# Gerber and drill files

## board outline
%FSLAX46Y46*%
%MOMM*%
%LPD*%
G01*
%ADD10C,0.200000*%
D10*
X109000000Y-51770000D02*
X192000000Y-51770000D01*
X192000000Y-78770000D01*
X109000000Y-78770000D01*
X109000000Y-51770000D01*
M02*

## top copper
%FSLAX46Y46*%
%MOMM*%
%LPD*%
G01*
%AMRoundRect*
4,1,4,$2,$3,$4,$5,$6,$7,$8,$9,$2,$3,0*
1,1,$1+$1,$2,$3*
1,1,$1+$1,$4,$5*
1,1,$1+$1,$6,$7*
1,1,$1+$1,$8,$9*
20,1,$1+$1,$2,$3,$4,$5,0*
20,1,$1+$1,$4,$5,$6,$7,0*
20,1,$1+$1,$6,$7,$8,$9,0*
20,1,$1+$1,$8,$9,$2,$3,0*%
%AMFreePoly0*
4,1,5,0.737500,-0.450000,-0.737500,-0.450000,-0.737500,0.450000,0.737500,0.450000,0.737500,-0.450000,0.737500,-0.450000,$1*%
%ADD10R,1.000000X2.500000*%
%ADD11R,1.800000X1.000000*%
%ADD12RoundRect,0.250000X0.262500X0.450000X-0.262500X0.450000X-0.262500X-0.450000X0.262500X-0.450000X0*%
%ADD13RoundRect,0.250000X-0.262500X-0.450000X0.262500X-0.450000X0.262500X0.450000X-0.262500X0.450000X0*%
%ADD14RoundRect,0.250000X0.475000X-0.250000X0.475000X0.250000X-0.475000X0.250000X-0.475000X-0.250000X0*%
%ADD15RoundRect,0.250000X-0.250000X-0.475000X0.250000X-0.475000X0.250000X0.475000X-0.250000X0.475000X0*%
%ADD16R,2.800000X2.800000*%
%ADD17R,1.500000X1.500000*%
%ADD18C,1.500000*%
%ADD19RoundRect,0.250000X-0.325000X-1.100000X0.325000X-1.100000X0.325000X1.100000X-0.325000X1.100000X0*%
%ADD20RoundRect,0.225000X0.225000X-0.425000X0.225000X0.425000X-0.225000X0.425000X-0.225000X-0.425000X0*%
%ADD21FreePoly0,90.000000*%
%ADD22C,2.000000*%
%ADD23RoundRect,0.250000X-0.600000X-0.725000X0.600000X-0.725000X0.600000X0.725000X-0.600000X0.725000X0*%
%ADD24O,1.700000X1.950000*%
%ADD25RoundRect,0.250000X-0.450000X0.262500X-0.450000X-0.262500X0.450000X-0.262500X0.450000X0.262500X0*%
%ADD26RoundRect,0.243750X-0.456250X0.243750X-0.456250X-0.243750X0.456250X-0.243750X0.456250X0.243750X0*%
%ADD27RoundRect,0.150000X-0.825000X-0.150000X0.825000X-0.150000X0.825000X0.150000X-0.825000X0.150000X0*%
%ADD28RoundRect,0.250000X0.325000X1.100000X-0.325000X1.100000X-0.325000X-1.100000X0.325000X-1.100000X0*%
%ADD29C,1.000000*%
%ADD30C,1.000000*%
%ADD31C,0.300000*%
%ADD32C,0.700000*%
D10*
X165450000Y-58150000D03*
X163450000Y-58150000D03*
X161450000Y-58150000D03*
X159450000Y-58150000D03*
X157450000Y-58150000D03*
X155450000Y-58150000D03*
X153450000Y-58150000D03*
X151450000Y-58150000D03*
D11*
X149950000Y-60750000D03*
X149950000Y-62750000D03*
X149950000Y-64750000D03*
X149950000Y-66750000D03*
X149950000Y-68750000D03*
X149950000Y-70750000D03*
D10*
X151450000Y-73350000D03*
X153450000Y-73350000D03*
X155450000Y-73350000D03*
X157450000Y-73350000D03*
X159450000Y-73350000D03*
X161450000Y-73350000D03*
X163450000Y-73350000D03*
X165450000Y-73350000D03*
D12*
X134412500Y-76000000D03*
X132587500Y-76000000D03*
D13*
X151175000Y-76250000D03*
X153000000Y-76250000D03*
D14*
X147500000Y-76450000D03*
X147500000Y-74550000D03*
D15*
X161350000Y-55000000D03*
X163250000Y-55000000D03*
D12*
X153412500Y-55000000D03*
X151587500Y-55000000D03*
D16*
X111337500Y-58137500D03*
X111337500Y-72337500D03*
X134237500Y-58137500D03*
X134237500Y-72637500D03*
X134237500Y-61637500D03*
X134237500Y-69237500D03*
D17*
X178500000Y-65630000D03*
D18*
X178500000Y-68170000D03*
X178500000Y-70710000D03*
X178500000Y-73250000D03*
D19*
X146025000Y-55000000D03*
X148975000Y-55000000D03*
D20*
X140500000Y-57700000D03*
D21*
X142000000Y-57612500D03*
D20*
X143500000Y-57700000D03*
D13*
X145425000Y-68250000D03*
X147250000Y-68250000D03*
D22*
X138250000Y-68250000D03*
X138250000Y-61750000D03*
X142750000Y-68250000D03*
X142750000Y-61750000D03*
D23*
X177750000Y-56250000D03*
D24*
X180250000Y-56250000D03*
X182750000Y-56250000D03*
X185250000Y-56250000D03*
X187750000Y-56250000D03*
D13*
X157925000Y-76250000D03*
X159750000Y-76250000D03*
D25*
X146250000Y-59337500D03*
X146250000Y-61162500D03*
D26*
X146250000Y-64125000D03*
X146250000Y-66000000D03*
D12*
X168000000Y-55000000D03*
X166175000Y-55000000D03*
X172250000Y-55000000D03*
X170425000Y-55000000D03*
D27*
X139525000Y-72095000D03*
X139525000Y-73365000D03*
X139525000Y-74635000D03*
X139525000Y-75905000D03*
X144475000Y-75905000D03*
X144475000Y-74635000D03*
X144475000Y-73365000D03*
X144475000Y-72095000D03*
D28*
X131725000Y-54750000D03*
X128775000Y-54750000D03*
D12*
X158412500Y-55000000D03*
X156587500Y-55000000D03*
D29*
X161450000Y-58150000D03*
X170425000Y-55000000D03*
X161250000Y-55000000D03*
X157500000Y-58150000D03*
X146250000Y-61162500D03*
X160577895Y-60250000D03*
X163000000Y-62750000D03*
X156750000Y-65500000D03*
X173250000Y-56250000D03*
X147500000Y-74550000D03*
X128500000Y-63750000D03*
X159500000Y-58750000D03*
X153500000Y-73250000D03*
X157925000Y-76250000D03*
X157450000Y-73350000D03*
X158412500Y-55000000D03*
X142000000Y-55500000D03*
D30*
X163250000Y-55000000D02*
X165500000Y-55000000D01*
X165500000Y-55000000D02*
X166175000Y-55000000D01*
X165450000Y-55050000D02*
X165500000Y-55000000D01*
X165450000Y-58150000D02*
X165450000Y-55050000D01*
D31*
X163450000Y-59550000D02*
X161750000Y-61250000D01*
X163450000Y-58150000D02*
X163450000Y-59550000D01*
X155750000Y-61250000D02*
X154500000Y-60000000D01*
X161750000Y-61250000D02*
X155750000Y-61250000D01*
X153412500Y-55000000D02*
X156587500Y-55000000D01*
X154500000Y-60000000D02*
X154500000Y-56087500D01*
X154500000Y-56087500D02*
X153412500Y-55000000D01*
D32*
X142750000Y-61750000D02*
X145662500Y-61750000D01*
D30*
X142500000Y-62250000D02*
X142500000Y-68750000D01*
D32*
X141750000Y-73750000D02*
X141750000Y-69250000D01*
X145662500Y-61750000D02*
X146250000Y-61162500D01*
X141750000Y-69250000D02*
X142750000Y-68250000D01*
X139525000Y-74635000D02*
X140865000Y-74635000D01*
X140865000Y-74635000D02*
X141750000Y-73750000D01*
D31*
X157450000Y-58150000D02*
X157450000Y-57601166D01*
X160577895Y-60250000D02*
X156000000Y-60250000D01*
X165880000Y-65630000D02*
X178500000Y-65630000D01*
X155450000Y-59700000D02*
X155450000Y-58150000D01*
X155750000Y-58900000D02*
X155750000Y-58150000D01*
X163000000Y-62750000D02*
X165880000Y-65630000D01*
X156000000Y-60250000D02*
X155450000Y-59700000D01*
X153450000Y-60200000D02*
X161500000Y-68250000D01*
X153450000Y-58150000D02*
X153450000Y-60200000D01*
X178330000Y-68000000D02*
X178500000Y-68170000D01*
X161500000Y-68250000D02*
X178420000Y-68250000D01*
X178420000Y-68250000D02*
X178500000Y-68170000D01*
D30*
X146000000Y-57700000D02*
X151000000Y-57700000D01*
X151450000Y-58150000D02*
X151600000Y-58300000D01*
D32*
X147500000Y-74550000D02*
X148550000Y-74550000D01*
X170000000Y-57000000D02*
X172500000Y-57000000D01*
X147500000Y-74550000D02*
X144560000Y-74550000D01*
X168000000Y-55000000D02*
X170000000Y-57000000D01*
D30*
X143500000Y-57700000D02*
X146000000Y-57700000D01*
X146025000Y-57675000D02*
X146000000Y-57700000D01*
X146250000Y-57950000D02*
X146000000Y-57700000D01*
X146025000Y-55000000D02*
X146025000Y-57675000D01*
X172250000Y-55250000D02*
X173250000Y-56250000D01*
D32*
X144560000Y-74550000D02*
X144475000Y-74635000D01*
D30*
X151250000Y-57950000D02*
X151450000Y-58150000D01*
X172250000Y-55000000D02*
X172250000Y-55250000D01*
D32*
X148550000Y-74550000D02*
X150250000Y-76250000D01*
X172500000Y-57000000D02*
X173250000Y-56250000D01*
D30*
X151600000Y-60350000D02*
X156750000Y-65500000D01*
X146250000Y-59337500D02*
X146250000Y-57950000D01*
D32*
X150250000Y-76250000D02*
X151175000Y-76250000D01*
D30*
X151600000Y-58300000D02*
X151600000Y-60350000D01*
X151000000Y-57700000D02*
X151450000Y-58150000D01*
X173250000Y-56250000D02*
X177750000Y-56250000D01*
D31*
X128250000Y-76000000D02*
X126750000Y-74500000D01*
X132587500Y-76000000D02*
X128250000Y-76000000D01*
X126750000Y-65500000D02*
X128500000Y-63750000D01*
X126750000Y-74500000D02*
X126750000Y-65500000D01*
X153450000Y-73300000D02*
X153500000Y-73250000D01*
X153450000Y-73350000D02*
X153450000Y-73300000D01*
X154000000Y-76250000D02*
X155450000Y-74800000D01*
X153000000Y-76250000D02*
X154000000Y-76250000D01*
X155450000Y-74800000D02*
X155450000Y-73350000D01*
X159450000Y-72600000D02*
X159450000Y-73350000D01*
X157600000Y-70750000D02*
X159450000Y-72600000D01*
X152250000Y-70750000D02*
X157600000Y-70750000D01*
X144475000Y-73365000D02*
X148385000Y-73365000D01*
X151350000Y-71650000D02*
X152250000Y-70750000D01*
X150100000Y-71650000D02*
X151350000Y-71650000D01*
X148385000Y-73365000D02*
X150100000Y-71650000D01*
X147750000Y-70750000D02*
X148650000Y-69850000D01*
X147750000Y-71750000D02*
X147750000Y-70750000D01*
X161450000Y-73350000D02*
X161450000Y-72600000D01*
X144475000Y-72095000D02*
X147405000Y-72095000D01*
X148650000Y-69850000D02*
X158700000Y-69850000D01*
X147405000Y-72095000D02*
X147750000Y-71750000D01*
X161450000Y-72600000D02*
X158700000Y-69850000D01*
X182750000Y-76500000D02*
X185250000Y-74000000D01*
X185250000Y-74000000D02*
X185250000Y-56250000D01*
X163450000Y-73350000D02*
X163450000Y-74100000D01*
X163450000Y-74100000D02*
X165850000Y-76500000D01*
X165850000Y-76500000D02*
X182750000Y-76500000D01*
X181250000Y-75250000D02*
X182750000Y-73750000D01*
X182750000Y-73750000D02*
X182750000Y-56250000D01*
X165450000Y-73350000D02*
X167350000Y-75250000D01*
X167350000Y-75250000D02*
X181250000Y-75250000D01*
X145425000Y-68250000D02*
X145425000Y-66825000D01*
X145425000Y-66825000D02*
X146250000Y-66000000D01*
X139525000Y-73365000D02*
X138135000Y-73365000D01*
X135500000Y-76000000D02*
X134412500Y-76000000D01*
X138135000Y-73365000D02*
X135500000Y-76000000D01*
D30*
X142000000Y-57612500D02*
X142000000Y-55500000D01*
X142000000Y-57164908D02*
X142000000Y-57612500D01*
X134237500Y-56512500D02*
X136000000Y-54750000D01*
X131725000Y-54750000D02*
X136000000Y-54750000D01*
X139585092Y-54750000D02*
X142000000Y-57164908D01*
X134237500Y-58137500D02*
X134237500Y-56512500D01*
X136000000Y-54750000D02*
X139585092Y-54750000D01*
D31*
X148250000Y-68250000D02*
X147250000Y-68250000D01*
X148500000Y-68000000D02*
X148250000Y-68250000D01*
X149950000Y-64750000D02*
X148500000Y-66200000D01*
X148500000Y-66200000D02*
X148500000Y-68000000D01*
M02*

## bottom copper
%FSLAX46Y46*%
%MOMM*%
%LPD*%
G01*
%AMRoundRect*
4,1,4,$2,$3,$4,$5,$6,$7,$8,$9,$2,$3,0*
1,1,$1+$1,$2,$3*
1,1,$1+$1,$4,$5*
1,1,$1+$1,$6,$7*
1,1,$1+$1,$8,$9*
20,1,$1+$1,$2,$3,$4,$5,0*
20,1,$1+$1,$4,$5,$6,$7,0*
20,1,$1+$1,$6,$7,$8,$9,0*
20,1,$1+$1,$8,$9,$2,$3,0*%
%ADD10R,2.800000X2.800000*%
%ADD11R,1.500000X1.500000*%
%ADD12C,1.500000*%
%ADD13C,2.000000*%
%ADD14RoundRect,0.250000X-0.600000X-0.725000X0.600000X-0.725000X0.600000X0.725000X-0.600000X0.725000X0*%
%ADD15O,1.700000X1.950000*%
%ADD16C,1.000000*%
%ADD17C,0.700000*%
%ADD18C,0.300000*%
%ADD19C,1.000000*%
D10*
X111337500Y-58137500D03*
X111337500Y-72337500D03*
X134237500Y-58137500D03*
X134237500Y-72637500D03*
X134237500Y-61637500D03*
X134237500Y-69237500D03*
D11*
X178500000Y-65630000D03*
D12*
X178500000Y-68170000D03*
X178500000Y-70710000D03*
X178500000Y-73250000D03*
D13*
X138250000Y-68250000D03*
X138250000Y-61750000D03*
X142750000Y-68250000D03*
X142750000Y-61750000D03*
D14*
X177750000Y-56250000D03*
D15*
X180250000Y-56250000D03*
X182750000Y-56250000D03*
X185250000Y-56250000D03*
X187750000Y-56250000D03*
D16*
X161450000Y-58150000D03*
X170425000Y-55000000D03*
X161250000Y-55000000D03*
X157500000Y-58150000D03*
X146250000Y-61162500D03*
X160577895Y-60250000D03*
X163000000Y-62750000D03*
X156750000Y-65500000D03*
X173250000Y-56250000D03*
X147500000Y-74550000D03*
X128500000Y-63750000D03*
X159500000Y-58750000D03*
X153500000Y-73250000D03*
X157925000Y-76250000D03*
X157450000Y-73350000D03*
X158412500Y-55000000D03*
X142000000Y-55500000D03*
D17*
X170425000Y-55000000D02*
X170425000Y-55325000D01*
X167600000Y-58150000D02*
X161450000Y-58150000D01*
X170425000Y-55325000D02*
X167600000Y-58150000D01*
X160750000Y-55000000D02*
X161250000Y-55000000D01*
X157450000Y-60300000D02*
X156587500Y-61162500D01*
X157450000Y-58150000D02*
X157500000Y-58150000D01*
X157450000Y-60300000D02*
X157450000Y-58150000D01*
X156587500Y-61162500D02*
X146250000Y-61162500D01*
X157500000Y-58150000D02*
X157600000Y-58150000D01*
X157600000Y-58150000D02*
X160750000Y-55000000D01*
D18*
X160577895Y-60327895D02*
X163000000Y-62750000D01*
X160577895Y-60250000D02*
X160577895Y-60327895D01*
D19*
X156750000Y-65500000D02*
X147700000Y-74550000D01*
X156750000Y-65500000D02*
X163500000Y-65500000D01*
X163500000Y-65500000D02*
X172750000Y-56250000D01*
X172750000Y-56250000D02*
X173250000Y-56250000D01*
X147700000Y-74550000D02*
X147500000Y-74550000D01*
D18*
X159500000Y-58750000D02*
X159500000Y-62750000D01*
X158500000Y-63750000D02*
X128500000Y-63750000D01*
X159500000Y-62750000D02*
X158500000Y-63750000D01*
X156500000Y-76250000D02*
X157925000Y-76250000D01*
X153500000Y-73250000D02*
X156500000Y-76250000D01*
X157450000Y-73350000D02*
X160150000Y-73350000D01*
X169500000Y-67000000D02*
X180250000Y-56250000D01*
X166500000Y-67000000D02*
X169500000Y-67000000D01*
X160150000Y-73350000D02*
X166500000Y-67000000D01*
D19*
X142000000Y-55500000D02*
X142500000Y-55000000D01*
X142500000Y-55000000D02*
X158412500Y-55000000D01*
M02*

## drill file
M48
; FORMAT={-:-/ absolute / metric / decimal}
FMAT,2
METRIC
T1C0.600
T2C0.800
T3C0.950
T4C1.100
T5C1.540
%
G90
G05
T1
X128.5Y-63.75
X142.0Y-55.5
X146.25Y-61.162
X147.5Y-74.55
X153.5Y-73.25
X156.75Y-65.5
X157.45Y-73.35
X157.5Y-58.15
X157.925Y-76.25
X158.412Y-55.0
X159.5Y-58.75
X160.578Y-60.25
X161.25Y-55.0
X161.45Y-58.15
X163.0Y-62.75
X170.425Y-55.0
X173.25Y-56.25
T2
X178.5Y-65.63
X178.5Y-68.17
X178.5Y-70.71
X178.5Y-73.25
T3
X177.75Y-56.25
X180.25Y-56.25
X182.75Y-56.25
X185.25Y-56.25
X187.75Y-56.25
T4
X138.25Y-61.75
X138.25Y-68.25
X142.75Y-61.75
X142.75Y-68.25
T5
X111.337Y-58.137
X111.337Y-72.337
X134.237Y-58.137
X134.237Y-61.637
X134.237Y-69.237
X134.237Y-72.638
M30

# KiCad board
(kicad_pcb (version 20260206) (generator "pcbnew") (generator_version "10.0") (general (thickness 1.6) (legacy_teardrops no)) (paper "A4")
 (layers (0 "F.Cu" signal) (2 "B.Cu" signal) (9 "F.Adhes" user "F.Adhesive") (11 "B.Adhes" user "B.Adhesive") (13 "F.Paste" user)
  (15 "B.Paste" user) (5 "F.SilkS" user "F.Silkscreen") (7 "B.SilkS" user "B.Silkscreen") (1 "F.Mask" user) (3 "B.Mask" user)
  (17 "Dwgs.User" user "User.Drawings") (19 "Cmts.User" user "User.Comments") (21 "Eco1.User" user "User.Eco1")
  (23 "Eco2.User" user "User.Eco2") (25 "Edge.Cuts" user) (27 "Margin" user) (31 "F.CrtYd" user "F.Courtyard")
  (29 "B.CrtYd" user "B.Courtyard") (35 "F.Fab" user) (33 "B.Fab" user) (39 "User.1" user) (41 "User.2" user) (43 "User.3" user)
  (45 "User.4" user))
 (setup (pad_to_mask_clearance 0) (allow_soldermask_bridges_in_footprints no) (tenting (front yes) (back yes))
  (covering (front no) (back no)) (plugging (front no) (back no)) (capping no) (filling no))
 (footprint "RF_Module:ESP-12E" (layer "F.Cu") (at 161.95 65.75 -90)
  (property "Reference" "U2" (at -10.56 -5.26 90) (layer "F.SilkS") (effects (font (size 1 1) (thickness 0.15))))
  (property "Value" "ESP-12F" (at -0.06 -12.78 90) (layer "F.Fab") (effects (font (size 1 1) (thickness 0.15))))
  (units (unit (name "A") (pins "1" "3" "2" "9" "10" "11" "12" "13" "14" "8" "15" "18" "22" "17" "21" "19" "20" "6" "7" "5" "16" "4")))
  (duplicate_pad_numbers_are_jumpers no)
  (pad "1" smd rect (at -7.6 -3.5 270) (size 2.5 1) (layers "F.Cu" "F.Mask" "F.Paste") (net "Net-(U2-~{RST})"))
  (pad "2" smd rect (at -7.6 -1.5 270) (size 2.5 1) (layers "F.Cu" "F.Mask" "F.Paste") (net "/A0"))
  (pad "3" smd rect (at -7.6 0.5 270) (size 2.5 1) (layers "F.Cu" "F.Mask" "F.Paste") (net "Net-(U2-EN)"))
  (pad "4" smd rect (at -7.6 2.5 270) (size 2.5 1) (layers "F.Cu" "F.Mask" "F.Paste") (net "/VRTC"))
  (pad "5" smd rect (at -7.6 4.5 270) (size 2.5 1) (layers "F.Cu" "F.Mask" "F.Paste") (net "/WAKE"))
  (pad "6" smd rect (at -7.6 6.5 270) (size 2.5 1) (layers "F.Cu" "F.Mask" "F.Paste") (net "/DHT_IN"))
  (pad "7" smd rect (at -7.6 8.5 270) (size 2.5 1) (layers "F.Cu" "F.Mask" "F.Paste") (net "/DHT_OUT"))
  (pad "8" smd rect (at -7.6 10.5 270) (size 2.5 1) (layers "F.Cu" "F.Mask" "F.Paste") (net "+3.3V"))
  (pad "9" smd rect (at -5 12 270) (size 1 1.8) (layers "F.Cu" "F.Mask" "F.Paste") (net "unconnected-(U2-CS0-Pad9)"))
  (pad "10" smd rect (at -3 12 270) (size 1 1.8) (layers "F.Cu" "F.Mask" "F.Paste") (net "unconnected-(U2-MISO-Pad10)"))
  (pad "11" smd rect (at -1 12 270) (size 1 1.8) (layers "F.Cu" "F.Mask" "F.Paste") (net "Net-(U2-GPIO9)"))
  (pad "12" smd rect (at 1 12 270) (size 1 1.8) (layers "F.Cu" "F.Mask" "F.Paste") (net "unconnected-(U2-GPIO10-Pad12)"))
  (pad "13" smd rect (at 3 12 270) (size 1 1.8) (layers "F.Cu" "F.Mask" "F.Paste") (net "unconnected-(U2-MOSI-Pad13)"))
  (pad "14" smd rect (at 5 12 270) (size 1 1.8) (layers "F.Cu" "F.Mask" "F.Paste") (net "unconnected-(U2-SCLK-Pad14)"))
  (pad "15" smd rect (at 7.6 10.5 270) (size 2.5 1) (layers "F.Cu" "F.Mask" "F.Paste") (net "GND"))
  (pad "16" smd rect (at 7.6 8.5 270) (size 2.5 1) (layers "F.Cu" "F.Mask" "F.Paste") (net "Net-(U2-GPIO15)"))
  (pad "17" smd rect (at 7.6 6.5 270) (size 2.5 1) (layers "F.Cu" "F.Mask" "F.Paste") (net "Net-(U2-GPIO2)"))
  (pad "18" smd rect (at 7.6 4.5 270) (size 2.5 1) (layers "F.Cu" "F.Mask" "F.Paste") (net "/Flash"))
  (pad "19" smd rect (at 7.6 2.5 270) (size 2.5 1) (layers "F.Cu" "F.Mask" "F.Paste") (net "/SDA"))
  (pad "20" smd rect (at 7.6 0.5 270) (size 2.5 1) (layers "F.Cu" "F.Mask" "F.Paste") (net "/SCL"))
  (pad "21" smd rect (at 7.6 -1.5 270) (size 2.5 1) (layers "F.Cu" "F.Mask" "F.Paste") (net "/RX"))
  (pad "22" smd rect (at 7.6 -3.5 270) (size 2.5 1) (layers "F.Cu" "F.Mask" "F.Paste") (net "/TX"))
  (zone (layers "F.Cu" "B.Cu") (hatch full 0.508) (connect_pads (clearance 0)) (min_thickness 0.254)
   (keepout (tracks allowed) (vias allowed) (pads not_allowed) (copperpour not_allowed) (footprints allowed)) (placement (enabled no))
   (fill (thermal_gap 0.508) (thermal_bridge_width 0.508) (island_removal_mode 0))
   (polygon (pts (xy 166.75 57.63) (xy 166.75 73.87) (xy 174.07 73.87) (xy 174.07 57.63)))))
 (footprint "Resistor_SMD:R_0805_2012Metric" (layer "F.Cu") (at 133.5 76 180)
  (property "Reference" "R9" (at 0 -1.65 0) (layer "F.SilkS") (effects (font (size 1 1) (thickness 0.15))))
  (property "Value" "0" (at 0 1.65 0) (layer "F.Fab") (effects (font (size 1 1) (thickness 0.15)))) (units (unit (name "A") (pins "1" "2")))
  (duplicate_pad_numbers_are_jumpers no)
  (pad "1" smd roundrect (at -0.9125 0 180) (size 1.025 1.4) (layers "F.Cu" "F.Mask" "F.Paste") (roundrect_rratio 0.243902)
   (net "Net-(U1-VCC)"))
  (pad "2" smd roundrect (at 0.9125 0 180) (size 1.025 1.4) (layers "F.Cu" "F.Mask" "F.Paste") (roundrect_rratio 0.243902) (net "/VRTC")))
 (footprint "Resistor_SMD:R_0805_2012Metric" (layer "F.Cu") (at 152.0875 76.25)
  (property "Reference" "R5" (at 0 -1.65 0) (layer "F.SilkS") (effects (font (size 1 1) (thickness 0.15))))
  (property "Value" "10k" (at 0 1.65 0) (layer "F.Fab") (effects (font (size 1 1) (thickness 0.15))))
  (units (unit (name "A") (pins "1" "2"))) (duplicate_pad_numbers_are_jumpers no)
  (pad "1" smd roundrect (at -0.9125 0) (size 1.025 1.4) (layers "F.Cu" "F.Mask" "F.Paste") (roundrect_rratio 0.243902) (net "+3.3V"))
  (pad "2" smd roundrect (at 0.9125 0) (size 1.025 1.4) (layers "F.Cu" "F.Mask" "F.Paste") (roundrect_rratio 0.243902)
   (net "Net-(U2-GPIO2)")))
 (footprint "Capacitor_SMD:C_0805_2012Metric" (layer "F.Cu") (at 147.5 75.5 90)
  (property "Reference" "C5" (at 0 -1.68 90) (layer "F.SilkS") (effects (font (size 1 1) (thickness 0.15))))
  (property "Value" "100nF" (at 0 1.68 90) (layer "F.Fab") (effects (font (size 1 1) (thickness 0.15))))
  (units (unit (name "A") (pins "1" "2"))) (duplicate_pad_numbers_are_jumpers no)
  (pad "1" smd roundrect (at -0.95 0 90) (size 1 1.45) (layers "F.Cu" "F.Mask" "F.Paste") (roundrect_rratio 0.25) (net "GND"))
  (pad "2" smd roundrect (at 0.95 0 90) (size 1 1.45) (layers "F.Cu" "F.Mask" "F.Paste") (roundrect_rratio 0.25) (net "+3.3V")))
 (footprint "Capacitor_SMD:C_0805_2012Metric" (layer "F.Cu") (at 162.3 55)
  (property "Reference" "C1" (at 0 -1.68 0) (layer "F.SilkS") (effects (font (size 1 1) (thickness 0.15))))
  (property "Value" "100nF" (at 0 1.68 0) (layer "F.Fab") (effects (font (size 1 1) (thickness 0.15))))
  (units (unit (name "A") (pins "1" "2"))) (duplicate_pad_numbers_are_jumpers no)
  (pad "1" smd roundrect (at -0.95 0) (size 1 1.45) (layers "F.Cu" "F.Mask" "F.Paste") (roundrect_rratio 0.25) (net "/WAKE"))
  (pad "2" smd roundrect (at 0.95 0) (size 1 1.45) (layers "F.Cu" "F.Mask" "F.Paste") (roundrect_rratio 0.25) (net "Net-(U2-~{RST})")))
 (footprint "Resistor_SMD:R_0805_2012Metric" (layer "F.Cu") (at 152.5 55 180)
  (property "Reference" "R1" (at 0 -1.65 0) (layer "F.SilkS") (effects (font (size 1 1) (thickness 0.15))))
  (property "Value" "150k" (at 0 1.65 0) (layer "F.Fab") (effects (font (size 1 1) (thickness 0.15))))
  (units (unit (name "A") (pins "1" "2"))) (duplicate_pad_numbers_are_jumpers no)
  (pad "1" smd roundrect (at -0.9125 0 180) (size 1.025 1.4) (layers "F.Cu" "F.Mask" "F.Paste") (roundrect_rratio 0.243902) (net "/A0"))
  (pad "2" smd roundrect (at 0.9125 0 180) (size 1.025 1.4) (layers "F.Cu" "F.Mask" "F.Paste") (roundrect_rratio 0.243902) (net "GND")))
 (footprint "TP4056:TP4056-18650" (layer "F.Cu") (at 109.6375 56.4375)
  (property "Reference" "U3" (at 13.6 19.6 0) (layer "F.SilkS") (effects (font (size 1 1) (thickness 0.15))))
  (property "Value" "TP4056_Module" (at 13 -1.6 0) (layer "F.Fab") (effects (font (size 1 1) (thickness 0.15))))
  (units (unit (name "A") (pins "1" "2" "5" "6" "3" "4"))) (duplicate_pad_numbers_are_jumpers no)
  (pad "1" thru_hole rect (at 1.7 1.7) (size 2.8 2.8) (drill 1.54) (layers "*.Cu" "*.Mask") (remove_unused_layers no)
   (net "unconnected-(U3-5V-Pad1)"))
  (pad "2" thru_hole rect (at 1.7 15.9) (size 2.8 2.8) (drill 1.54) (layers "*.Cu" "*.Mask") (remove_unused_layers no)
   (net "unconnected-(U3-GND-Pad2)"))
  (pad "3" thru_hole rect (at 24.6 1.7) (size 2.8 2.8) (drill 1.54) (layers "*.Cu" "*.Mask") (remove_unused_layers no) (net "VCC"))
  (pad "4" thru_hole rect (at 24.6 16.2) (size 2.8 2.8) (drill 1.54) (layers "*.Cu" "*.Mask") (remove_unused_layers no) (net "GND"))
  (pad "5" thru_hole rect (at 24.6 5.2) (size 2.8 2.8) (drill 1.54) (layers "*.Cu" "*.Mask") (remove_unused_layers no) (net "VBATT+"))
  (pad "6" thru_hole rect (at 24.6 12.8) (size 2.8 2.8) (drill 1.54) (layers "*.Cu" "*.Mask") (remove_unused_layers no) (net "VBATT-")))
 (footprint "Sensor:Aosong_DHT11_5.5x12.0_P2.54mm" (layer "F.Cu") (at 178.5 65.63)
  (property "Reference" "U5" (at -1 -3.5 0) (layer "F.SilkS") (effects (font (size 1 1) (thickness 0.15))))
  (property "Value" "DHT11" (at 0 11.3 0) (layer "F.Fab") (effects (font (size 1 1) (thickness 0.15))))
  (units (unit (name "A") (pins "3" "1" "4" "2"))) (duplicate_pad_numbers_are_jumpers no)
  (pad "1" thru_hole rect (at 0 0) (size 1.5 1.5) (drill 0.8) (layers "*.Cu" "*.Mask") (remove_unused_layers no) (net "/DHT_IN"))
  (pad "2" thru_hole circle (at 0 2.54) (size 1.5 1.5) (drill 0.8) (layers "*.Cu" "*.Mask") (remove_unused_layers no) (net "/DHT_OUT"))
  (pad "3" thru_hole circle (at 0 5.08) (size 1.5 1.5) (drill 0.8) (layers "*.Cu" "*.Mask") (remove_unused_layers no)
   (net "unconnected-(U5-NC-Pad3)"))
  (pad "4" thru_hole circle (at 0 7.62) (size 1.5 1.5) (drill 0.8) (layers "*.Cu" "*.Mask") (remove_unused_layers no) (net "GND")))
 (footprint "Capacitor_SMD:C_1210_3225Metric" (layer "F.Cu") (at 147.5 55)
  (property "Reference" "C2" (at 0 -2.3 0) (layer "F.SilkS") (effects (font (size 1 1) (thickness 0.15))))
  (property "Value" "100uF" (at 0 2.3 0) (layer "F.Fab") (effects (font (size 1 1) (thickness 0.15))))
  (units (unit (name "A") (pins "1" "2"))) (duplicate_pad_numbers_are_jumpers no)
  (pad "1" smd roundrect (at -1.475 0) (size 1.15 2.7) (layers "F.Cu" "F.Mask" "F.Paste") (roundrect_rratio 0.217391) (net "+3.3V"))
  (pad "2" smd roundrect (at 1.475 0) (size 1.15 2.7) (layers "F.Cu" "F.Mask" "F.Paste") (roundrect_rratio 0.217391) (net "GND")))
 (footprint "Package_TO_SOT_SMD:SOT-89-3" (layer "F.Cu") (at 142 55.75 90)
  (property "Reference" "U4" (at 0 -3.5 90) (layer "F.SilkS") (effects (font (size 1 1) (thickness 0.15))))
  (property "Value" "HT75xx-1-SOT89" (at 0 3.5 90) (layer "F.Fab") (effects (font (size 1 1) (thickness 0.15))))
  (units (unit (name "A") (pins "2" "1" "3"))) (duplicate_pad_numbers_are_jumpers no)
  (pad "1" smd roundrect (at -1.95 -1.5 90) (size 1.3 0.9) (layers "F.Cu" "F.Mask" "F.Paste") (roundrect_rratio 0.25) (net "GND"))
  (pad "2" smd custom (at -1.8625 0 90) (size 1.475 0.9) (layers "F.Cu" "F.Mask" "F.Paste") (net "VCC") (zone_connect 2)
   (thermal_bridge_angle 45) (options (clearance outline) (anchor rect)) (primitives))
  (pad "3" smd roundrect (at -1.95 1.5 90) (size 1.3 0.9) (layers "F.Cu" "F.Mask" "F.Paste") (roundrect_rratio 0.25) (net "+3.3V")))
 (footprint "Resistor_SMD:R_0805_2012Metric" (layer "F.Cu") (at 146.3375 68.25)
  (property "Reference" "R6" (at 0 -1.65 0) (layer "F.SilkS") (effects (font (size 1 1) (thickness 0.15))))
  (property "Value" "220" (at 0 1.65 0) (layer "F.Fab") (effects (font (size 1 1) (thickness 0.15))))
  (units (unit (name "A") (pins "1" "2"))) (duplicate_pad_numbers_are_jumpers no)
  (pad "1" smd roundrect (at -0.9125 0) (size 1.025 1.4) (layers "F.Cu" "F.Mask" "F.Paste") (roundrect_rratio 0.243902) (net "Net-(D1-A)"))
  (pad "2" smd roundrect (at 0.9125 0) (size 1.025 1.4) (layers "F.Cu" "F.Mask" "F.Paste") (roundrect_rratio 0.243902)
   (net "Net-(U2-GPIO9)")))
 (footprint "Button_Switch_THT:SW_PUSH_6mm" (layer "F.Cu") (at 138.25 68.25 90)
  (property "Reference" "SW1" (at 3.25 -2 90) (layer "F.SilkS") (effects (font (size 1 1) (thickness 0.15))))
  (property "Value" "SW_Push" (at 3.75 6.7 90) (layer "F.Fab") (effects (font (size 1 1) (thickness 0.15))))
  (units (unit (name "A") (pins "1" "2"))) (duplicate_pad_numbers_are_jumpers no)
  (pad "1" thru_hole circle (at 0 0 180) (size 2 2) (drill 1.1) (layers "*.Cu" "*.Mask") (remove_unused_layers no) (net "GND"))
  (pad "1" thru_hole circle (at 6.5 0 180) (size 2 2) (drill 1.1) (layers "*.Cu" "*.Mask") (remove_unused_layers no) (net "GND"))
  (pad "2" thru_hole circle (at 0 4.5 180) (size 2 2) (drill 1.1) (layers "*.Cu" "*.Mask") (remove_unused_layers no) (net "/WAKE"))
  (pad "2" thru_hole circle (at 6.5 4.5 180) (size 2 2) (drill 1.1) (layers "*.Cu" "*.Mask") (remove_unused_layers no) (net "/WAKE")))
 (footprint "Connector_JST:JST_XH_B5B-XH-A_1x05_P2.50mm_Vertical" (layer "F.Cu") (at 177.75 56.25)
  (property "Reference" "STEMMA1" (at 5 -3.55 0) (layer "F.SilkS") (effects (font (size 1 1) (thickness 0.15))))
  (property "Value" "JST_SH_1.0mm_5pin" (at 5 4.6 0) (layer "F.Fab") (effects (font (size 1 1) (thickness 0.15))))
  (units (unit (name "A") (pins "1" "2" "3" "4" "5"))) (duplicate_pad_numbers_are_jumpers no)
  (pad "1" thru_hole roundrect (at 0 0) (size 1.7 1.95) (drill 0.95) (layers "*.Cu" "*.Mask") (remove_unused_layers no)
   (roundrect_rratio 0.147059) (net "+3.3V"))
  (pad "2" thru_hole oval (at 2.5 0) (size 1.7 1.95) (drill 0.95) (layers "*.Cu" "*.Mask") (remove_unused_layers no) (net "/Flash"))
  (pad "3" thru_hole oval (at 5 0) (size 1.7 1.95) (drill 0.95) (layers "*.Cu" "*.Mask") (remove_unused_layers no) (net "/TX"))
  (pad "4" thru_hole oval (at 7.5 0) (size 1.7 1.95) (drill 0.95) (layers "*.Cu" "*.Mask") (remove_unused_layers no) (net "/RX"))
  (pad "5" thru_hole oval (at 10 0) (size 1.7 1.95) (drill 0.95) (layers "*.Cu" "*.Mask") (remove_unused_layers no) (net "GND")))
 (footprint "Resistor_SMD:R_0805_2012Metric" (layer "F.Cu") (at 158.8375 76.25)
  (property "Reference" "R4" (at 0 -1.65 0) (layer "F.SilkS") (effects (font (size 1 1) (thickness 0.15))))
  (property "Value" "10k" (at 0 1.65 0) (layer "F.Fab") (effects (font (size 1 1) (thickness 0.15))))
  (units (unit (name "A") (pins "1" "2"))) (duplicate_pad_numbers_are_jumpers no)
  (pad "1" smd roundrect (at -0.9125 0) (size 1.025 1.4) (layers "F.Cu" "F.Mask" "F.Paste") (roundrect_rratio 0.243902)
   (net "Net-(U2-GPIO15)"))
  (pad "2" smd roundrect (at 0.9125 0) (size 1.025 1.4) (layers "F.Cu" "F.Mask" "F.Paste") (roundrect_rratio 0.243902) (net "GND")))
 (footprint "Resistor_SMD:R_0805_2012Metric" (layer "F.Cu") (at 146.25 60.25 -90)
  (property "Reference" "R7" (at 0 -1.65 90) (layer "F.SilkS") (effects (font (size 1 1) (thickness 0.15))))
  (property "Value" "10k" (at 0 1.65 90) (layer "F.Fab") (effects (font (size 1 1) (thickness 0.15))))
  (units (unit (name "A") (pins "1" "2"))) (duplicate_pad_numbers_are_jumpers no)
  (pad "1" smd roundrect (at -0.9125 0 270) (size 1.025 1.4) (layers "F.Cu" "F.Mask" "F.Paste") (roundrect_rratio 0.243902) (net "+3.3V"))
  (pad "2" smd roundrect (at 0.9125 0 270) (size 1.025 1.4) (layers "F.Cu" "F.Mask" "F.Paste") (roundrect_rratio 0.243902) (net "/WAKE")))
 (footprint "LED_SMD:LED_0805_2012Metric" (layer "F.Cu") (at 146.25 65.0625 -90)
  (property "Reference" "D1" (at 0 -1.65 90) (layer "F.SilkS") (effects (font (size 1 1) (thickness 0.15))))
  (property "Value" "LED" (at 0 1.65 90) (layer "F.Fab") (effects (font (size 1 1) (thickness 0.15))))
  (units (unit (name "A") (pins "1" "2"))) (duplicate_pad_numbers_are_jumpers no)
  (pad "1" smd roundrect (at -0.9375 0 270) (size 0.975 1.4) (layers "F.Cu" "F.Mask" "F.Paste") (roundrect_rratio 0.25) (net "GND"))
  (pad "2" smd roundrect (at 0.9375 0 270) (size 0.975 1.4) (layers "F.Cu" "F.Mask" "F.Paste") (roundrect_rratio 0.25) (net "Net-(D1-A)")))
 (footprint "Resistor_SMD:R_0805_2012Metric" (layer "F.Cu") (at 167.0875 55 180)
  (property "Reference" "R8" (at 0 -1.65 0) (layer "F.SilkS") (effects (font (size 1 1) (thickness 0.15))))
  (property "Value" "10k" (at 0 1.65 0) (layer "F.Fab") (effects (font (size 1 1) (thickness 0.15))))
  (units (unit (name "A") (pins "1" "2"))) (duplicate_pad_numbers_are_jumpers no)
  (pad "1" smd roundrect (at -0.9125 0 180) (size 1.025 1.4) (layers "F.Cu" "F.Mask" "F.Paste") (roundrect_rratio 0.243902) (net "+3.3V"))
  (pad "2" smd roundrect (at 0.9125 0 180) (size 1.025 1.4) (layers "F.Cu" "F.Mask" "F.Paste") (roundrect_rratio 0.243902)
   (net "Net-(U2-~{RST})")))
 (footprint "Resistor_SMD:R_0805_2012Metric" (layer "F.Cu") (at 171.3375 55 180)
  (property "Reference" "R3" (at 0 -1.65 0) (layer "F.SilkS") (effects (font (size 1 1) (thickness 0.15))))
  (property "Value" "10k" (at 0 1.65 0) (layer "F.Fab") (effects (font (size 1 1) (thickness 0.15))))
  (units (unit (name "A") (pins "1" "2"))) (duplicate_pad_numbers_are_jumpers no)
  (pad "1" smd roundrect (at -0.9125 0 180) (size 1.025 1.4) (layers "F.Cu" "F.Mask" "F.Paste") (roundrect_rratio 0.243902) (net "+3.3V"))
  (pad "2" smd roundrect (at 0.9125 0 180) (size 1.025 1.4) (layers "F.Cu" "F.Mask" "F.Paste") (roundrect_rratio 0.243902)
   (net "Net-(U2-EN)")))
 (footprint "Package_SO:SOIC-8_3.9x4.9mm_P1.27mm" (layer "F.Cu") (at 142 74)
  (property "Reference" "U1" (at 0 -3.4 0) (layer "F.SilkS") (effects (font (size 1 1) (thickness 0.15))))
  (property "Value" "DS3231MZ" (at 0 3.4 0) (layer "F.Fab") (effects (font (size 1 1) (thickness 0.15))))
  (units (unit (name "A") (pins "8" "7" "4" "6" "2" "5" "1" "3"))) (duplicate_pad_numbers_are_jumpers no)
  (pad "1" smd roundrect (at -2.475 -1.905) (size 1.95 0.6) (layers "F.Cu" "F.Mask" "F.Paste") (roundrect_rratio 0.25)
   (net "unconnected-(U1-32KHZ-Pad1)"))
  (pad "2" smd roundrect (at -2.475 -0.635) (size 1.95 0.6) (layers "F.Cu" "F.Mask" "F.Paste") (roundrect_rratio 0.25) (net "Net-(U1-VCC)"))
  (pad "3" smd roundrect (at -2.475 0.635) (size 1.95 0.6) (layers "F.Cu" "F.Mask" "F.Paste") (roundrect_rratio 0.25) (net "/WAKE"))
  (pad "4" smd roundrect (at -2.475 1.905) (size 1.95 0.6) (layers "F.Cu" "F.Mask" "F.Paste") (roundrect_rratio 0.25)
   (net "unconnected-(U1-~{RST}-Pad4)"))
  (pad "5" smd roundrect (at 2.475 1.905) (size 1.95 0.6) (layers "F.Cu" "F.Mask" "F.Paste") (roundrect_rratio 0.25) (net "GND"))
  (pad "6" smd roundrect (at 2.475 0.635) (size 1.95 0.6) (layers "F.Cu" "F.Mask" "F.Paste") (roundrect_rratio 0.25) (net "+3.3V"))
  (pad "7" smd roundrect (at 2.475 -0.635) (size 1.95 0.6) (layers "F.Cu" "F.Mask" "F.Paste") (roundrect_rratio 0.25) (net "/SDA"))
  (pad "8" smd roundrect (at 2.475 -1.905) (size 1.95 0.6) (layers "F.Cu" "F.Mask" "F.Paste") (roundrect_rratio 0.25) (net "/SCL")))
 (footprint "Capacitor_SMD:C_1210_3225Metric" (layer "F.Cu") (at 130.25 54.75 180)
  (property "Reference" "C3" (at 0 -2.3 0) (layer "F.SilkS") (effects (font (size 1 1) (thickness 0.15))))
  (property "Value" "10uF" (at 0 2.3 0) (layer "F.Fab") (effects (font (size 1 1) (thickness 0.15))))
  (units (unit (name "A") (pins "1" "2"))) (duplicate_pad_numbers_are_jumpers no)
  (pad "1" smd roundrect (at -1.475 0 180) (size 1.15 2.7) (layers "F.Cu" "F.Mask" "F.Paste") (roundrect_rratio 0.217391) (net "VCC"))
  (pad "2" smd roundrect (at 1.475 0 180) (size 1.15 2.7) (layers "F.Cu" "F.Mask" "F.Paste") (roundrect_rratio 0.217391) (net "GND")))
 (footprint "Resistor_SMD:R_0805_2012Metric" (layer "F.Cu") (at 157.5 55 180)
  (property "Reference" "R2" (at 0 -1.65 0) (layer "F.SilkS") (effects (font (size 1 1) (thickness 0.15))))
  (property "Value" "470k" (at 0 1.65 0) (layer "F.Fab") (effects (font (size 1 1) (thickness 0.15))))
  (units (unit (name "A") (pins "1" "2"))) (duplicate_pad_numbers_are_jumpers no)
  (pad "1" smd roundrect (at -0.9125 0 180) (size 1.025 1.4) (layers "F.Cu" "F.Mask" "F.Paste") (roundrect_rratio 0.243902) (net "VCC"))
  (pad "2" smd roundrect (at 0.9125 0 180) (size 1.025 1.4) (layers "F.Cu" "F.Mask" "F.Paste") (roundrect_rratio 0.243902) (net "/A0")))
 (gr_rect (start 109 51.77) (end 192 78.77) (stroke (width 0.2) (type solid)) (fill no) (layer "Edge.Cuts"))
 (segment (start 163.25 55) (end 165.5 55) (width 1) (layer "F.Cu") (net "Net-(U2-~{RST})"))
 (segment (start 165.5 55) (end 166.175 55) (width 1) (layer "F.Cu") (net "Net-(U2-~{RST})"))
 (segment (start 165.45 55.05) (end 165.5 55) (width 1) (layer "F.Cu") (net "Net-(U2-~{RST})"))
 (segment (start 165.45 58.15) (end 165.45 55.05) (width 1) (layer "F.Cu") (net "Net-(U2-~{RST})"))
 (segment (start 163.45 59.55) (end 161.75 61.25) (width 0.3) (layer "F.Cu") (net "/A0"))
 (segment (start 163.45 58.15) (end 163.45 59.55) (width 0.3) (layer "F.Cu") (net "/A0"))
 (segment (start 155.75 61.25) (end 154.5 60) (width 0.3) (layer "F.Cu") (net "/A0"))
 (segment (start 161.75 61.25) (end 155.75 61.25) (width 0.3) (layer "F.Cu") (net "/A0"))
 (segment (start 153.4125 55) (end 156.5875 55) (width 0.3) (layer "F.Cu") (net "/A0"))
 (segment (start 154.5 60) (end 154.5 56.0875) (width 0.3) (layer "F.Cu") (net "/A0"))
 (segment (start 154.5 56.0875) (end 153.4125 55) (width 0.3) (layer "F.Cu") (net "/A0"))
 (via (at 161.45 58.15) (size 1) (drill 0.6) (layers "F.Cu" "B.Cu") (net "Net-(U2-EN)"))
 (via (at 170.425 55) (size 1) (drill 0.6) (layers "F.Cu" "B.Cu") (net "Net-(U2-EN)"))
 (segment (start 170.425 55) (end 170.425 55.325) (width 0.7) (layer "B.Cu") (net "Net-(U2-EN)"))
 (segment (start 167.6 58.15) (end 161.45 58.15) (width 0.7) (layer "B.Cu") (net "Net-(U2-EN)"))
 (segment (start 170.425 55.325) (end 167.6 58.15) (width 0.7) (layer "B.Cu") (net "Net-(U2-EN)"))
 (segment (start 142.75 61.75) (end 145.6625 61.75) (width 0.7) (layer "F.Cu") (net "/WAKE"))
 (segment (start 142.5 62.25) (end 142.5 68.75) (width 1) (layer "F.Cu") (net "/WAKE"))
 (segment (start 141.75 73.75) (end 141.75 69.25) (width 0.7) (layer "F.Cu") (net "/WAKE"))
 (segment (start 145.6625 61.75) (end 146.25 61.1625) (width 0.7) (layer "F.Cu") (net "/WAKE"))
 (segment (start 141.75 69.25) (end 142.75 68.25) (width 0.7) (layer "F.Cu") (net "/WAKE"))
 (segment (start 139.525 74.635) (end 140.865 74.635) (width 0.7) (layer "F.Cu") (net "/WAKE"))
 (segment (start 140.865 74.635) (end 141.75 73.75) (width 0.7) (layer "F.Cu") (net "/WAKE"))
 (segment (start 157.45 58.15) (end 157.45 57.601166) (width 0.3) (layer "F.Cu") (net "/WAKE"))
 (via (at 161.25 55) (size 1) (drill 0.6) (layers "F.Cu" "B.Cu") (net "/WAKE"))
 (via (at 157.5 58.15) (size 1) (drill 0.6) (layers "F.Cu" "B.Cu") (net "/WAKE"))
 (via (at 146.25 61.1625) (size 1) (drill 0.6) (layers "F.Cu" "B.Cu") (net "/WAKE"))
 (segment (start 160.75 55) (end 161.25 55) (width 0.7) (layer "B.Cu") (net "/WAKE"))
 (segment (start 157.45 60.3) (end 156.5875 61.1625) (width 0.7) (layer "B.Cu") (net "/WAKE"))
 (segment (start 157.45 58.15) (end 157.5 58.15) (width 0.7) (layer "B.Cu") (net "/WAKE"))
 (segment (start 157.45 60.3) (end 157.45 58.15) (width 0.7) (layer "B.Cu") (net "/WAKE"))
 (segment (start 156.5875 61.1625) (end 146.25 61.1625) (width 0.7) (layer "B.Cu") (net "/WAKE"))
 (segment (start 157.5 58.15) (end 157.6 58.15) (width 0.7) (layer "B.Cu") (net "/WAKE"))
 (segment (start 157.6 58.15) (end 160.75 55) (width 0.7) (layer "B.Cu") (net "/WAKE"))
 (segment (start 160.577895 60.25) (end 156 60.25) (width 0.3) (layer "F.Cu") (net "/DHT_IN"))
 (segment (start 165.88 65.63) (end 178.5 65.63) (width 0.3) (layer "F.Cu") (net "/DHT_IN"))
 (segment (start 155.45 59.7) (end 155.45 58.15) (width 0.3) (layer "F.Cu") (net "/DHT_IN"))
 (segment (start 155.75 58.9) (end 155.75 58.15) (width 0.3) (layer "F.Cu") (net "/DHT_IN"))
 (segment (start 163 62.75) (end 165.88 65.63) (width 0.3) (layer "F.Cu") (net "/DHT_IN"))
 (segment (start 156 60.25) (end 155.45 59.7) (width 0.3) (layer "F.Cu") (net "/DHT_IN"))
 (via (at 160.577895 60.25) (size 1) (drill 0.6) (layers "F.Cu" "B.Cu") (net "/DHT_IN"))
 (via (at 163 62.75) (size 1) (drill 0.6) (layers "F.Cu" "B.Cu") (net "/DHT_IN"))
 (segment (start 160.577895 60.327895) (end 163 62.75) (width 0.3) (layer "B.Cu") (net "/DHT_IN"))
 (segment (start 160.577895 60.25) (end 160.577895 60.327895) (width 0.3) (layer "B.Cu") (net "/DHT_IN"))
 (segment (start 153.45 60.2) (end 161.5 68.25) (width 0.3) (layer "F.Cu") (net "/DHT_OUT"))
 (segment (start 153.45 58.15) (end 153.45 60.2) (width 0.3) (layer "F.Cu") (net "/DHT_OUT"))
 (segment (start 178.33 68) (end 178.5 68.17) (width 0.3) (layer "F.Cu") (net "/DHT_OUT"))
 (segment (start 161.5 68.25) (end 178.42 68.25) (width 0.3) (layer "F.Cu") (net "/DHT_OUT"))
 (segment (start 178.42 68.25) (end 178.5 68.17) (width 0.3) (layer "F.Cu") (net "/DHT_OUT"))
 (segment (start 146 57.7) (end 151 57.7) (width 1) (layer "F.Cu") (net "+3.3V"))
 (segment (start 151.45 58.15) (end 151.6 58.3) (width 1) (layer "F.Cu") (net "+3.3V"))
 (segment (start 147.5 74.55) (end 148.55 74.55) (width 0.7) (layer "F.Cu") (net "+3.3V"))
 (segment (start 170 57) (end 172.5 57) (width 0.7) (layer "F.Cu") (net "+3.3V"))
 (segment (start 147.5 74.55) (end 144.56 74.55) (width 0.7) (layer "F.Cu") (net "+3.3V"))
 (segment (start 168 55) (end 170 57) (width 0.7) (layer "F.Cu") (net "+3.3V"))
 (segment (start 143.5 57.7) (end 146 57.7) (width 1) (layer "F.Cu") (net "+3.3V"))
 (segment (start 146.025 57.675) (end 146 57.7) (width 1) (layer "F.Cu") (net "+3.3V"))
 (segment (start 146.25 57.95) (end 146 57.7) (width 1) (layer "F.Cu") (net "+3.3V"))
 (segment (start 146.025 55) (end 146.025 57.675) (width 1) (layer "F.Cu") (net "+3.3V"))
 (segment (start 172.25 55.25) (end 173.25 56.25) (width 1) (layer "F.Cu") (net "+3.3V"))
 (segment (start 144.56 74.55) (end 144.475 74.635) (width 0.7) (layer "F.Cu") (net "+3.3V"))
 (segment (start 151.25 57.95) (end 151.45 58.15) (width 1) (layer "F.Cu") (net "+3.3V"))
 (segment (start 172.25 55) (end 172.25 55.25) (width 1) (layer "F.Cu") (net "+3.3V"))
 (segment (start 148.55 74.55) (end 150.25 76.25) (width 0.7) (layer "F.Cu") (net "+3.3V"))
 (segment (start 172.5 57) (end 173.25 56.25) (width 0.7) (layer "F.Cu") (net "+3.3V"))
 (segment (start 151.6 60.35) (end 156.75 65.5) (width 1) (layer "F.Cu") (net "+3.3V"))
 (segment (start 146.25 59.3375) (end 146.25 57.95) (width 1) (layer "F.Cu") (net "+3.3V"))
 (segment (start 150.25 76.25) (end 151.175 76.25) (width 0.7) (layer "F.Cu") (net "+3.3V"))
 (segment (start 151.6 58.3) (end 151.6 60.35) (width 1) (layer "F.Cu") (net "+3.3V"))
 (segment (start 151 57.7) (end 151.45 58.15) (width 1) (layer "F.Cu") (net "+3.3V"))
 (segment (start 173.25 56.25) (end 177.75 56.25) (width 1) (layer "F.Cu") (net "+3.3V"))
 (via (at 156.75 65.5) (size 1) (drill 0.6) (layers "F.Cu" "B.Cu") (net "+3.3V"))
 (via (at 173.25 56.25) (size 1) (drill 0.6) (layers "F.Cu" "B.Cu") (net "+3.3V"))
 (via (at 147.5 74.55) (size 1) (drill 0.6) (layers "F.Cu" "B.Cu") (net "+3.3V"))
 (segment (start 156.75 65.5) (end 147.7 74.55) (width 1) (layer "B.Cu") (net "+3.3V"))
 (segment (start 156.75 65.5) (end 163.5 65.5) (width 1) (layer "B.Cu") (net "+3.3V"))
 (segment (start 163.5 65.5) (end 172.75 56.25) (width 1) (layer "B.Cu") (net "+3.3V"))
 (segment (start 172.75 56.25) (end 173.25 56.25) (width 1) (layer "B.Cu") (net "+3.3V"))
 (segment (start 147.7 74.55) (end 147.5 74.55) (width 1) (layer "B.Cu") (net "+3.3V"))
 (segment (start 128.25 76) (end 126.75 74.5) (width 0.3) (layer "F.Cu") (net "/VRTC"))
 (segment (start 132.5875 76) (end 128.25 76) (width 0.3) (layer "F.Cu") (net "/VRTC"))
 (segment (start 126.75 65.5) (end 128.5 63.75) (width 0.3) (layer "F.Cu") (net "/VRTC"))
 (segment (start 126.75 74.5) (end 126.75 65.5) (width 0.3) (layer "F.Cu") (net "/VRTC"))
 (via (at 128.5 63.75) (size 1) (drill 0.6) (layers "F.Cu" "B.Cu") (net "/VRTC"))
 (via (at 159.5 58.75) (size 1) (drill 0.6) (layers "F.Cu" "B.Cu") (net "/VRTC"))
 (segment (start 159.5 58.75) (end 159.5 62.75) (width 0.3) (layer "B.Cu") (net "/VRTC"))
 (segment (start 158.5 63.75) (end 128.5 63.75) (width 0.3) (layer "B.Cu") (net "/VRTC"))
 (segment (start 159.5 62.75) (end 158.5 63.75) (width 0.3) (layer "B.Cu") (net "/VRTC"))
 (segment (start 153.45 73.3) (end 153.5 73.25) (width 0.3) (layer "F.Cu") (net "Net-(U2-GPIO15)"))
 (segment (start 153.45 73.35) (end 153.45 73.3) (width 0.3) (layer "F.Cu") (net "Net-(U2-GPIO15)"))
 (via (at 153.5 73.25) (size 1) (drill 0.6) (layers "F.Cu" "B.Cu") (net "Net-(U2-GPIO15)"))
 (via (at 157.925 76.25) (size 1) (drill 0.6) (layers "F.Cu" "B.Cu") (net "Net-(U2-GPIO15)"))
 (segment (start 156.5 76.25) (end 157.925 76.25) (width 0.3) (layer "B.Cu") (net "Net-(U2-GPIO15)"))
 (segment (start 153.5 73.25) (end 156.5 76.25) (width 0.3) (layer "B.Cu") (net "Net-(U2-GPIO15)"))
 (segment (start 154 76.25) (end 155.45 74.8) (width 0.3) (layer "F.Cu") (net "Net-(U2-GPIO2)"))
 (segment (start 153 76.25) (end 154 76.25) (width 0.3) (layer "F.Cu") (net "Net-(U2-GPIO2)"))
 (segment (start 155.45 74.8) (end 155.45 73.35) (width 0.3) (layer "F.Cu") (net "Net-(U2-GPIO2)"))
 (via (at 157.45 73.35) (size 1) (drill 0.6) (layers "F.Cu" "B.Cu") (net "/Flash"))
 (segment (start 157.45 73.35) (end 160.15 73.35) (width 0.3) (layer "B.Cu") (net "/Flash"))
 (segment (start 169.5 67) (end 180.25 56.25) (width 0.3) (layer "B.Cu") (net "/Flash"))
 (segment (start 166.5 67) (end 169.5 67) (width 0.3) (layer "B.Cu") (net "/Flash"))
 (segment (start 160.15 73.35) (end 166.5 67) (width 0.3) (layer "B.Cu") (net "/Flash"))
 (segment (start 159.45 72.6) (end 159.45 73.35) (width 0.3) (layer "F.Cu") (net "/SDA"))
 (segment (start 157.6 70.75) (end 159.45 72.6) (width 0.3) (layer "F.Cu") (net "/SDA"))
 (segment (start 152.25 70.75) (end 157.6 70.75) (width 0.3) (layer "F.Cu") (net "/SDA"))
 (segment (start 144.475 73.365) (end 148.385 73.365) (width 0.3) (layer "F.Cu") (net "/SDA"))
 (segment (start 151.35 71.65) (end 152.25 70.75) (width 0.3) (layer "F.Cu") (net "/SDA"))
 (segment (start 150.1 71.65) (end 151.35 71.65) (width 0.3) (layer "F.Cu") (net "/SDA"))
 (segment (start 148.385 73.365) (end 150.1 71.65) (width 0.3) (layer "F.Cu") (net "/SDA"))
 (segment (start 147.75 70.75) (end 148.65 69.85) (width 0.3) (layer "F.Cu") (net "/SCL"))
 (segment (start 147.75 71.75) (end 147.75 70.75) (width 0.3) (layer "F.Cu") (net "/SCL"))
 (segment (start 161.45 73.35) (end 161.45 72.6) (width 0.3) (layer "F.Cu") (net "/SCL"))
 (segment (start 144.475 72.095) (end 147.405 72.095) (width 0.3) (layer "F.Cu") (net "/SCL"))
 (segment (start 148.65 69.85) (end 158.7 69.85) (width 0.3) (layer "F.Cu") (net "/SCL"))
 (segment (start 147.405 72.095) (end 147.75 71.75) (width 0.3) (layer "F.Cu") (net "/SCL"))
 (segment (start 161.45 72.6) (end 158.7 69.85) (width 0.3) (layer "F.Cu") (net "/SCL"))
 (segment (start 182.75 76.5) (end 185.25 74) (width 0.3) (layer "F.Cu") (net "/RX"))
 (segment (start 185.25 74) (end 185.25 56.25) (width 0.3) (layer "F.Cu") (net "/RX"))
 (segment (start 163.45 73.35) (end 163.45 74.1) (width 0.3) (layer "F.Cu") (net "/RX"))
 (segment (start 163.45 74.1) (end 165.85 76.5) (width 0.3) (layer "F.Cu") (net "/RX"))
 (segment (start 165.85 76.5) (end 182.75 76.5) (width 0.3) (layer "F.Cu") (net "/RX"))
 (segment (start 181.25 75.25) (end 182.75 73.75) (width 0.3) (layer "F.Cu") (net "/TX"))
 (segment (start 182.75 73.75) (end 182.75 56.25) (width 0.3) (layer "F.Cu") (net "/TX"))
 (segment (start 165.45 73.35) (end 167.35 75.25) (width 0.3) (layer "F.Cu") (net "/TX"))
 (segment (start 167.35 75.25) (end 181.25 75.25) (width 0.3) (layer "F.Cu") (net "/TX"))
 (segment (start 145.425 68.25) (end 145.425 66.825) (width 0.3) (layer "F.Cu") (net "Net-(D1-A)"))
 (segment (start 145.425 66.825) (end 146.25 66) (width 0.3) (layer "F.Cu") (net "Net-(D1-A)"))
 (segment (start 139.525 73.365) (end 138.135 73.365) (width 0.3) (layer "F.Cu") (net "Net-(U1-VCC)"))
 (segment (start 135.5 76) (end 134.4125 76) (width 0.3) (layer "F.Cu") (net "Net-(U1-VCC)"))
 (segment (start 138.135 73.365) (end 135.5 76) (width 0.3) (layer "F.Cu") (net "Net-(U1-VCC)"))
 (segment (start 142 57.6125) (end 142 55.5) (width 1) (layer "F.Cu") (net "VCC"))
 (segment (start 142 57.164908) (end 142 57.6125) (width 1) (layer "F.Cu") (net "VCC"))
 (segment (start 134.2375 56.5125) (end 136 54.75) (width 1) (layer "F.Cu") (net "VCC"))
 (segment (start 131.725 54.75) (end 136 54.75) (width 1) (layer "F.Cu") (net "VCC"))
 (segment (start 139.585092 54.75) (end 142 57.164908) (width 1) (layer "F.Cu") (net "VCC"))
 (segment (start 134.2375 58.1375) (end 134.2375 56.5125) (width 1) (layer "F.Cu") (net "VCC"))
 (segment (start 136 54.75) (end 139.585092 54.75) (width 1) (layer "F.Cu") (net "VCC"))
 (via (at 158.4125 55) (size 1) (drill 0.6) (layers "F.Cu" "B.Cu") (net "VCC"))
 (via (at 142 55.5) (size 1) (drill 0.6) (layers "F.Cu" "B.Cu") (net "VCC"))
 (segment (start 142 55.5) (end 142.5 55) (width 1) (layer "B.Cu") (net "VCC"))
 (segment (start 142.5 55) (end 158.4125 55) (width 1) (layer "B.Cu") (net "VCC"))
 (segment (start 148.25 68.25) (end 147.25 68.25) (width 0.3) (layer "F.Cu") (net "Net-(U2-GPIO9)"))
 (segment (start 148.5 68) (end 148.25 68.25) (width 0.3) (layer "F.Cu") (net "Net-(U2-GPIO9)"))
 (segment (start 149.95 64.75) (end 148.5 66.2) (width 0.3) (layer "F.Cu") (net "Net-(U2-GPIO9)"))
 (segment (start 148.5 66.2) (end 148.5 68) (width 0.3) (layer "F.Cu") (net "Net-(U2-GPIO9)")))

